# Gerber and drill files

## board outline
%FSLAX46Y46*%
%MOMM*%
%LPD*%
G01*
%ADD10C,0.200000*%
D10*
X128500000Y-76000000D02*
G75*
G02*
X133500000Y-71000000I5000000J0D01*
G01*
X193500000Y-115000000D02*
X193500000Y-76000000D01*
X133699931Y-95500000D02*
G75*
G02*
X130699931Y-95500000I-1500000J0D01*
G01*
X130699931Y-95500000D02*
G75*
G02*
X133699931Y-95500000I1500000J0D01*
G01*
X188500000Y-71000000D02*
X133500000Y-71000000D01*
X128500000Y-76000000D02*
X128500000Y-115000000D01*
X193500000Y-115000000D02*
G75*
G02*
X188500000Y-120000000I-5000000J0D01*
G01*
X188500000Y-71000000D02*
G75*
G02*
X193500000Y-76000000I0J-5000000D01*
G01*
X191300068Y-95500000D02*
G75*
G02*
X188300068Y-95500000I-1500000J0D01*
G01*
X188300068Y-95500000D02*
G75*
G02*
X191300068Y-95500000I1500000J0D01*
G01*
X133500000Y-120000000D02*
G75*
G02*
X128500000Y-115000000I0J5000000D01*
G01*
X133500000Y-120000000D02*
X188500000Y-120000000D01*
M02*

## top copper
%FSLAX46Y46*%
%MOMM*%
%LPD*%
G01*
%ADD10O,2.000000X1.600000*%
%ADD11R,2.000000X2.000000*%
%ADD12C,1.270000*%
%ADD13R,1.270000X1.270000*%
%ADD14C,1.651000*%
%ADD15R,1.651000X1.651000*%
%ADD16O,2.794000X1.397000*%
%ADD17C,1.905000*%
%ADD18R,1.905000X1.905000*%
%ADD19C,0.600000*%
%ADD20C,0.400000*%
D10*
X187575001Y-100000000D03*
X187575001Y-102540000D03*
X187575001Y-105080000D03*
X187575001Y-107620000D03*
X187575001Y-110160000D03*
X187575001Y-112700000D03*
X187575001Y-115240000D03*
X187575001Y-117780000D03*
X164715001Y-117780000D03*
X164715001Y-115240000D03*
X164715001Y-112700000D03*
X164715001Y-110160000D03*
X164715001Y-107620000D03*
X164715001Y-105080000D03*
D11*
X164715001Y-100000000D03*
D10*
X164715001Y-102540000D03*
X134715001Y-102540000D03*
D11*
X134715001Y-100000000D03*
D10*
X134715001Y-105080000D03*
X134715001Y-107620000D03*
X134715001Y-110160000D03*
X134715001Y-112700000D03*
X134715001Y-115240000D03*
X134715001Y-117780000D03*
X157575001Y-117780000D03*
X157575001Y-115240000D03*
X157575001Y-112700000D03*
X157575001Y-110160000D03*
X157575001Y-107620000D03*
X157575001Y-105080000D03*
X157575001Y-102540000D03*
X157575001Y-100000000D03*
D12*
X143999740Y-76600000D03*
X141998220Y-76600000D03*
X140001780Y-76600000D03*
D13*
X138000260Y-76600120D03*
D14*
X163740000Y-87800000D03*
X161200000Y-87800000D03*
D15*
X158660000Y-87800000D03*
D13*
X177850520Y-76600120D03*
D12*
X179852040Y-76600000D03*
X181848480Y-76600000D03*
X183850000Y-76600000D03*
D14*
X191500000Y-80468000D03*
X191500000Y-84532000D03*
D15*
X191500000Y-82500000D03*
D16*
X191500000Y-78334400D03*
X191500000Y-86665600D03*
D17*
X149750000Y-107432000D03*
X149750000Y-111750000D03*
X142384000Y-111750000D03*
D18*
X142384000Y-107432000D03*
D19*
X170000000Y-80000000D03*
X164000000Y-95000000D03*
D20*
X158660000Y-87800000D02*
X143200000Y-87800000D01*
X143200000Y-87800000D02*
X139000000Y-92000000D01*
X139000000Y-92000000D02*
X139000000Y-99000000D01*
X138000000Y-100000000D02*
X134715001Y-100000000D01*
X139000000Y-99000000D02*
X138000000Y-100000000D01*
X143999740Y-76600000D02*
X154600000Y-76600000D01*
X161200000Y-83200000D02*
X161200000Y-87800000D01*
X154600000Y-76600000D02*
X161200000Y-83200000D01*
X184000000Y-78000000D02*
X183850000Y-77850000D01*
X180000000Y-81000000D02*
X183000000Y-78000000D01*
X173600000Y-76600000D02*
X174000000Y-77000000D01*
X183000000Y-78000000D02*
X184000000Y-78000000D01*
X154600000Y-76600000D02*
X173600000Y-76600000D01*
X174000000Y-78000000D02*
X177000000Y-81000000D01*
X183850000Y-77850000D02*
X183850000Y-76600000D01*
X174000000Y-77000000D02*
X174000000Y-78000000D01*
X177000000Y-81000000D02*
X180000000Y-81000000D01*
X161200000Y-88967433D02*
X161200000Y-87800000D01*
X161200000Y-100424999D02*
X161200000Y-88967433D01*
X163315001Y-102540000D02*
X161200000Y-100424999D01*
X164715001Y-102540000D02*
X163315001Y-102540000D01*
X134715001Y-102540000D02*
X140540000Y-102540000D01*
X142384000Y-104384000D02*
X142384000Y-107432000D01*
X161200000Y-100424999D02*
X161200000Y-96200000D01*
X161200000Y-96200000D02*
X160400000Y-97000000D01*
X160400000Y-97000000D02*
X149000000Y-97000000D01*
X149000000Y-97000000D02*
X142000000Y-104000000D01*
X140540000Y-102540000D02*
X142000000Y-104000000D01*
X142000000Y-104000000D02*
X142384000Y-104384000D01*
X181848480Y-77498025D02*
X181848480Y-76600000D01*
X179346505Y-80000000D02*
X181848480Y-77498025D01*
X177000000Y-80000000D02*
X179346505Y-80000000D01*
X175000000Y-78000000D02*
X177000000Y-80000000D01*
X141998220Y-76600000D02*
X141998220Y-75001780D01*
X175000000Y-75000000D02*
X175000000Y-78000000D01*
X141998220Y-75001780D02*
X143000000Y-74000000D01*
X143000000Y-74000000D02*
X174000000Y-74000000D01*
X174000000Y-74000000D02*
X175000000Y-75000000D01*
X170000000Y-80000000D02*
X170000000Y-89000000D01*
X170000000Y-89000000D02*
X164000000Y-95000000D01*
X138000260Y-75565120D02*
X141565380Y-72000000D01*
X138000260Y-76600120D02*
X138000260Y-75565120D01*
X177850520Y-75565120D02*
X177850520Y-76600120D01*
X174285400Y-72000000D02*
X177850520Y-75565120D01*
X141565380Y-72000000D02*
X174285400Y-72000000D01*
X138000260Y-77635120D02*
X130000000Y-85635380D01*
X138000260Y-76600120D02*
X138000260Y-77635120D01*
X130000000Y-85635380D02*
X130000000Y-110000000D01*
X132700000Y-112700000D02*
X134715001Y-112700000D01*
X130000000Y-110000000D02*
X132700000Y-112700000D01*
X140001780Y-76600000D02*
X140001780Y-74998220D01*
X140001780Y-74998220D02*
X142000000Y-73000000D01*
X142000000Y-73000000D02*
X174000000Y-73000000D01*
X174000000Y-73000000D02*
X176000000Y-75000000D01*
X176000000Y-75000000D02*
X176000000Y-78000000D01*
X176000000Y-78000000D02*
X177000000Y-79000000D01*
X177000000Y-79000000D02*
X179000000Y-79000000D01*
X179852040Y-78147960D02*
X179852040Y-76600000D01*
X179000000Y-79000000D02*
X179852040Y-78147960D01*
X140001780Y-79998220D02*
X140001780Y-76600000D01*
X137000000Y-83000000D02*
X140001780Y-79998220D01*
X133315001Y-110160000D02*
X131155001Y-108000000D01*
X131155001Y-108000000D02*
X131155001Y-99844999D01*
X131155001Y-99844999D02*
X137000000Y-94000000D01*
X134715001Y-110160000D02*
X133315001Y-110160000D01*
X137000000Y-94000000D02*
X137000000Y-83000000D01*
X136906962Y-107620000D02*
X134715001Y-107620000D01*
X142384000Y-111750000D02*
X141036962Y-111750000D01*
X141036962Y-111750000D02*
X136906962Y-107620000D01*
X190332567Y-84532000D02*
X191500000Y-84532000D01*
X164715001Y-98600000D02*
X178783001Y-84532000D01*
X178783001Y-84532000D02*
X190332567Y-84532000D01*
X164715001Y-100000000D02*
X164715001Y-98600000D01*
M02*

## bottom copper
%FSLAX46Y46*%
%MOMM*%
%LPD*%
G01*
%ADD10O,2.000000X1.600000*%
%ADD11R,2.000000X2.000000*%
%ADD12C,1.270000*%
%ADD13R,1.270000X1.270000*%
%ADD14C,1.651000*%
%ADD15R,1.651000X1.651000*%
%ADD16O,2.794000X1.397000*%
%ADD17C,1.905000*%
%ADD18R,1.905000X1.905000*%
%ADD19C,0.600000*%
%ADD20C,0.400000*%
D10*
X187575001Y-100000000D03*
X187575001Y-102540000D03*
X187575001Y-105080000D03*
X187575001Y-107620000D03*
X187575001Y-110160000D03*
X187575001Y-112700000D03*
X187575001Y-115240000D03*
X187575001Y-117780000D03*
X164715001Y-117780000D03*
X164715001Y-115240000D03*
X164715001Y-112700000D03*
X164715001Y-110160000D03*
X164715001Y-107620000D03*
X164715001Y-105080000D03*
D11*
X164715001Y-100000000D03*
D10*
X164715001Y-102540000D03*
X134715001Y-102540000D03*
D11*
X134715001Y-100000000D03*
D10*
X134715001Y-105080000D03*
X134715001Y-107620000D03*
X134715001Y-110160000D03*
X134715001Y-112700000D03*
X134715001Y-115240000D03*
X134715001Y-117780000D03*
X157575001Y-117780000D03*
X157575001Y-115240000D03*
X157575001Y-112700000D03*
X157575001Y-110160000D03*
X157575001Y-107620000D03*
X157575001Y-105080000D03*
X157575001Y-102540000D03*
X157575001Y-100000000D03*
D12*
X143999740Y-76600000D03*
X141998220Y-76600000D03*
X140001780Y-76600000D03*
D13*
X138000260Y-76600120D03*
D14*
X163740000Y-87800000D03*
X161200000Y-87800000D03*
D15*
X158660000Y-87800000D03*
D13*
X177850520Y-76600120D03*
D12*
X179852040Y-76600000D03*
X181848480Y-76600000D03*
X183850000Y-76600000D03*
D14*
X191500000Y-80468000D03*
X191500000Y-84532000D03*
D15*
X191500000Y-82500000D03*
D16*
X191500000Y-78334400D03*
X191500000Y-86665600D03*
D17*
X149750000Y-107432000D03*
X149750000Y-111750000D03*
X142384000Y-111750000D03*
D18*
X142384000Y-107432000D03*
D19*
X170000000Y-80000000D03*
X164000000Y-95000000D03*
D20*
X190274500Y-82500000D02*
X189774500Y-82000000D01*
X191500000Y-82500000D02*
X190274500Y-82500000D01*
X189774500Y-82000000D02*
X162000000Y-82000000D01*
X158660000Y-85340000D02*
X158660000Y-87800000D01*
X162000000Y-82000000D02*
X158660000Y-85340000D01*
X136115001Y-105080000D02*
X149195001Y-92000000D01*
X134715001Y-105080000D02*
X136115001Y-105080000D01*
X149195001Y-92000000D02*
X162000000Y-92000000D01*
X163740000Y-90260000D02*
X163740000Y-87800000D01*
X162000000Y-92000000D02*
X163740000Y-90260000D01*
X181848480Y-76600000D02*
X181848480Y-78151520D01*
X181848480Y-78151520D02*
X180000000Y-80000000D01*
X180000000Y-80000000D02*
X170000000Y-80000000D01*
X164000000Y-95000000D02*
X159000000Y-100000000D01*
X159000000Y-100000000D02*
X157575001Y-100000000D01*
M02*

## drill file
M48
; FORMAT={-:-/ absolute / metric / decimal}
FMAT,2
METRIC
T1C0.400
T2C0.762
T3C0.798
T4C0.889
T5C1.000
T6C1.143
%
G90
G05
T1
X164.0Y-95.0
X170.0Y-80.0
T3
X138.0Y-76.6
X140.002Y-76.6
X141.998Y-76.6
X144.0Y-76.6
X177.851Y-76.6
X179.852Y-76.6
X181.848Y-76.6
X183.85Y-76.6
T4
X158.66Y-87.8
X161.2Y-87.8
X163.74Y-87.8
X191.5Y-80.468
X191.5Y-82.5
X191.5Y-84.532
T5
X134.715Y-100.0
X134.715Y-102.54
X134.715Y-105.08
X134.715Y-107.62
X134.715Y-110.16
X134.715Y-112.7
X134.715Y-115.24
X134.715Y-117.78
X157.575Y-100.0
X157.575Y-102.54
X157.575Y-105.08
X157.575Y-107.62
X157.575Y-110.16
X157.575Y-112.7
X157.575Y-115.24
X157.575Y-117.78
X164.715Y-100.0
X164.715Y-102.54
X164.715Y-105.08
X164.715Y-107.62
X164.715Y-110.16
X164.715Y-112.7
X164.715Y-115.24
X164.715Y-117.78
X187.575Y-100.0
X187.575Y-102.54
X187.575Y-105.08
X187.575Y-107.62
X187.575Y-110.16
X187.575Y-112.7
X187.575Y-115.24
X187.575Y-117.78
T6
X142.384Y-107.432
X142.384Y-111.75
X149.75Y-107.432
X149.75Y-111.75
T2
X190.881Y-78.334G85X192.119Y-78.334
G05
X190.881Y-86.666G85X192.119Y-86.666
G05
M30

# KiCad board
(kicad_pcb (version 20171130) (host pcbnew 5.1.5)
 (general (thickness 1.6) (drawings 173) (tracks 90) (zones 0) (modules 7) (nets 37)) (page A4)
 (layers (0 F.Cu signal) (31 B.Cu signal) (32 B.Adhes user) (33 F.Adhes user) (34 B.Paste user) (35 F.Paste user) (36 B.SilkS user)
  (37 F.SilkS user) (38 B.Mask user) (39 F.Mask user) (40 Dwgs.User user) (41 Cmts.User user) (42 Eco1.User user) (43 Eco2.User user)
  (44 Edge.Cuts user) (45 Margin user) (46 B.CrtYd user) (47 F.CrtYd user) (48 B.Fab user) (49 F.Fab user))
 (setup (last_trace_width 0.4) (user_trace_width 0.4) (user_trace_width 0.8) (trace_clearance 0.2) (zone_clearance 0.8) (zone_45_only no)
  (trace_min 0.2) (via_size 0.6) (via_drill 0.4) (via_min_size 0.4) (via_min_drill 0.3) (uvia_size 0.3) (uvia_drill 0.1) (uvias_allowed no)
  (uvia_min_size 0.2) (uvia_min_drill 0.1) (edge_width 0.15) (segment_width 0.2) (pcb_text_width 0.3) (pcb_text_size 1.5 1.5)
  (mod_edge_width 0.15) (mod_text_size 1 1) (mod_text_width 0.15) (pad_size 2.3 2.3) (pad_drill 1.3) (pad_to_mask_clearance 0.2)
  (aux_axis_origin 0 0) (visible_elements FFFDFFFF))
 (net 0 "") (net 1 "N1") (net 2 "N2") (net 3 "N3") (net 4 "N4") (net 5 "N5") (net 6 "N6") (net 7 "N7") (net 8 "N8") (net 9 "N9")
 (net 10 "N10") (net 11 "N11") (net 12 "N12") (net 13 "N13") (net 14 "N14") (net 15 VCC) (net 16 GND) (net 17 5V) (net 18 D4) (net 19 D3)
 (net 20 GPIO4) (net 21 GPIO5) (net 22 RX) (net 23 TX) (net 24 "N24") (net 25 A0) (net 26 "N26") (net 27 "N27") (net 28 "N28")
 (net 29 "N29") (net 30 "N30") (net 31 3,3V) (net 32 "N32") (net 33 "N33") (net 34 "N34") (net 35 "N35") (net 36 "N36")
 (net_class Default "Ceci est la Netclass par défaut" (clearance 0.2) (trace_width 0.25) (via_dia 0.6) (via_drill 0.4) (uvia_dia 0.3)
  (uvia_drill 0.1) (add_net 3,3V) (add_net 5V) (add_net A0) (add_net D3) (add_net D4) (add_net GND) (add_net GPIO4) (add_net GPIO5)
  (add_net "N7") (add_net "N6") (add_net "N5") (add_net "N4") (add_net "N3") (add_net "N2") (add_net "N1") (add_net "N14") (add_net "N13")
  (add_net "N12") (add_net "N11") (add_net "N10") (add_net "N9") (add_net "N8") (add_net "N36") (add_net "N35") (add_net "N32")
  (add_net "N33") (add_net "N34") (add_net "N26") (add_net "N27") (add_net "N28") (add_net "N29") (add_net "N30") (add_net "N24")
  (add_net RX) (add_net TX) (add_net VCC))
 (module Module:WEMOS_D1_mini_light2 (layer F.Cu) (at 164.715001 100)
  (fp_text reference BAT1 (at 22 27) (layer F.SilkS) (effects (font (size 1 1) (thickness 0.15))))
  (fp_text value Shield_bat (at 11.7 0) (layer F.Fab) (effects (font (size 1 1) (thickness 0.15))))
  (pad 16 thru_hole oval (at 22.86 0) (size 2 1.6) (drill 1) (layers *.Cu *.Mask) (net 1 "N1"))
  (pad 15 thru_hole oval (at 22.86 2.54) (size 2 1.6) (drill 1) (layers *.Cu *.Mask) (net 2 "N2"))
  (pad 14 thru_hole oval (at 22.86 5.08) (size 2 1.6) (drill 1) (layers *.Cu *.Mask) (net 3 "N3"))
  (pad 13 thru_hole oval (at 22.86 7.62) (size 2 1.6) (drill 1) (layers *.Cu *.Mask) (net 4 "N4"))
  (pad 12 thru_hole oval (at 22.86 10.16) (size 2 1.6) (drill 1) (layers *.Cu *.Mask) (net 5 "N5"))
  (pad 11 thru_hole oval (at 22.86 12.7) (size 2 1.6) (drill 1) (layers *.Cu *.Mask) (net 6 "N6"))
  (pad 10 thru_hole oval (at 22.86 15.24) (size 2 1.6) (drill 1) (layers *.Cu *.Mask) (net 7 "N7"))
  (pad 9 thru_hole oval (at 22.86 17.78) (size 2 1.6) (drill 1) (layers *.Cu *.Mask) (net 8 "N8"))
  (pad 8 thru_hole oval (at 0 17.78) (size 2 1.6) (drill 1) (layers *.Cu *.Mask) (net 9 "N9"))
  (pad 7 thru_hole oval (at 0 15.24) (size 2 1.6) (drill 1) (layers *.Cu *.Mask) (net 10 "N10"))
  (pad 6 thru_hole oval (at 0 12.7) (size 2 1.6) (drill 1) (layers *.Cu *.Mask) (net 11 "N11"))
  (pad 5 thru_hole oval (at 0 10.16) (size 2 1.6) (drill 1) (layers *.Cu *.Mask) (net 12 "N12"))
  (pad 4 thru_hole oval (at 0 7.62) (size 2 1.6) (drill 1) (layers *.Cu *.Mask) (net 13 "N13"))
  (pad 3 thru_hole oval (at 0 5.08) (size 2 1.6) (drill 1) (layers *.Cu *.Mask) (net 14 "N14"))
  (pad 1 thru_hole rect (at 0 0) (size 2 2) (drill 1) (layers *.Cu *.Mask) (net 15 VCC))
  (pad 2 thru_hole oval (at 0 2.54) (size 2 1.6) (drill 1) (layers *.Cu *.Mask) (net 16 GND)))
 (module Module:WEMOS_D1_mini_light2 (layer F.Cu) (at 134.715001 100)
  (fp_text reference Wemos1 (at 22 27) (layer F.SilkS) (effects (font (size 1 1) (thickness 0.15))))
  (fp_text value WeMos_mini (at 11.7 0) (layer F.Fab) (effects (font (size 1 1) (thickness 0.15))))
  (pad 2 thru_hole oval (at 0 2.54) (size 2 1.6) (drill 1) (layers *.Cu *.Mask) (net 16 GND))
  (pad 1 thru_hole rect (at 0 0) (size 2 2) (drill 1) (layers *.Cu *.Mask) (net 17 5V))
  (pad 3 thru_hole oval (at 0 5.08) (size 2 1.6) (drill 1) (layers *.Cu *.Mask) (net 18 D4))
  (pad 4 thru_hole oval (at 0 7.62) (size 2 1.6) (drill 1) (layers *.Cu *.Mask) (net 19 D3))
  (pad 5 thru_hole oval (at 0 10.16) (size 2 1.6) (drill 1) (layers *.Cu *.Mask) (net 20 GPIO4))
  (pad 6 thru_hole oval (at 0 12.7) (size 2 1.6) (drill 1) (layers *.Cu *.Mask) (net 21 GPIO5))
  (pad 7 thru_hole oval (at 0 15.24) (size 2 1.6) (drill 1) (layers *.Cu *.Mask) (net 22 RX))
  (pad 8 thru_hole oval (at 0 17.78) (size 2 1.6) (drill 1) (layers *.Cu *.Mask) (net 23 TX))
  (pad 9 thru_hole oval (at 22.86 17.78) (size 2 1.6) (drill 1) (layers *.Cu *.Mask) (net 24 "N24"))
  (pad 10 thru_hole oval (at 22.86 15.24) (size 2 1.6) (drill 1) (layers *.Cu *.Mask) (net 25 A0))
  (pad 11 thru_hole oval (at 22.86 12.7) (size 2 1.6) (drill 1) (layers *.Cu *.Mask) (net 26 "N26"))
  (pad 12 thru_hole oval (at 22.86 10.16) (size 2 1.6) (drill 1) (layers *.Cu *.Mask) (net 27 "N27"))
  (pad 13 thru_hole oval (at 22.86 7.62) (size 2 1.6) (drill 1) (layers *.Cu *.Mask) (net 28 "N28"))
  (pad 14 thru_hole oval (at 22.86 5.08) (size 2 1.6) (drill 1) (layers *.Cu *.Mask) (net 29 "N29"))
  (pad 15 thru_hole oval (at 22.86 2.54) (size 2 1.6) (drill 1) (layers *.Cu *.Mask) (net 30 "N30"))
  (pad 16 thru_hole oval (at 22.86 0) (size 2 1.6) (drill 1) (layers *.Cu *.Mask) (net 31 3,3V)))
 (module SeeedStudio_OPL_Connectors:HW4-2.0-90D (layer F.Cu) (at 141 73.4)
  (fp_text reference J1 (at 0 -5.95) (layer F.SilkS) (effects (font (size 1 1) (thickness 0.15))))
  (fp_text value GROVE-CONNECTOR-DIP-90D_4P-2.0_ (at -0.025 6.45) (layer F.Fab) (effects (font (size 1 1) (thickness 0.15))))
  (pad 4 thru_hole circle (at 2.99974 3.2) (size 1.27 1.27) (drill 0.79756) (layers *.Cu *.Mask) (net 16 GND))
  (pad 3 thru_hole circle (at 0.99822 3.2) (size 1.27 1.27) (drill 0.79756) (layers *.Cu *.Mask) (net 31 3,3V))
  (pad 2 thru_hole circle (at -0.99822 3.2) (size 1.27 1.27) (drill 0.79756) (layers *.Cu *.Mask) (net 20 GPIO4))
  (pad 1 thru_hole rect (at -2.99974 3.20012) (size 1.27 1.27) (drill 0.79756) (layers *.Cu *.Mask) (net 21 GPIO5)))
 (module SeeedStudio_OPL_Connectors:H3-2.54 (layer F.Cu) (at 161.2 87.8 180)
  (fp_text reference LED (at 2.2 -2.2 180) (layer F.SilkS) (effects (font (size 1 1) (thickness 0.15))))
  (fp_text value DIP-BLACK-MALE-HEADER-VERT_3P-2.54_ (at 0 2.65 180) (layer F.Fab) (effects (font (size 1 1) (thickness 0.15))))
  (pad 3 thru_hole circle (at -2.54 0 270) (size 1.651 1.651) (drill 0.889) (layers *.Cu *.Mask) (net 18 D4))
  (pad 2 thru_hole circle (at 0 0 270) (size 1.651 1.651) (drill 0.889) (layers *.Cu *.Mask) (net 16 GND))
  (pad 1 thru_hole rect (at 2.54 0 270) (size 1.651 1.651) (drill 0.889) (layers *.Cu *.Mask) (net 17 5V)))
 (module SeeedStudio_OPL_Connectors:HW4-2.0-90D (layer F.Cu) (at 180.85026 73.4)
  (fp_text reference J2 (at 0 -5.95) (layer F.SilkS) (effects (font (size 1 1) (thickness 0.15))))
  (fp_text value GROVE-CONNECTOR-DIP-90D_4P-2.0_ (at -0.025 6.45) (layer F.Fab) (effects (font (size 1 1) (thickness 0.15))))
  (pad 1 thru_hole rect (at -2.99974 3.20012) (size 1.27 1.27) (drill 0.79756) (layers *.Cu *.Mask) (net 21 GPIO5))
  (pad 2 thru_hole circle (at -0.99822 3.2) (size 1.27 1.27) (drill 0.79756) (layers *.Cu *.Mask) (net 20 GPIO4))
  (pad 3 thru_hole circle (at 0.99822 3.2) (size 1.27 1.27) (drill 0.79756) (layers *.Cu *.Mask) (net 31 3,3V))
  (pad 4 thru_hole circle (at 2.99974 3.2) (size 1.27 1.27) (drill 0.79756) (layers *.Cu *.Mask) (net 16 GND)))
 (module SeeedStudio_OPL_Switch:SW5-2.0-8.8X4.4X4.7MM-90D (layer F.Cu) (at 191.5 82.5)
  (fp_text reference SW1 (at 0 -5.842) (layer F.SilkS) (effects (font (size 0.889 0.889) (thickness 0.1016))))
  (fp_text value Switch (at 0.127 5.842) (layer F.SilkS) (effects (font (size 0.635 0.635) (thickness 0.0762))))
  (pad A thru_hole circle (at 0 -2.032) (size 1.651 1.651) (drill 0.889) (layers *.Cu *.Mask) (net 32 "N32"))
  (pad B thru_hole circle (at 0 2.032) (size 1.651 1.651) (drill 0.889) (layers *.Cu *.Mask) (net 15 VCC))
  (pad COM thru_hole rect (at 0 0) (size 1.651 1.651) (drill 0.889) (layers *.Cu *.Mask) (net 17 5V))
  (pad NC1 thru_hole oval (at 0 -4.1656 90) (size 1.397 2.794) (drill oval 0.762 2) (layers *.Cu *.Mask) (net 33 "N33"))
  (pad NC2 thru_hole oval (at 0 4.1656 90) (size 1.397 2.794) (drill oval 0.762 2) (layers *.Cu *.Mask) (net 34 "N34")))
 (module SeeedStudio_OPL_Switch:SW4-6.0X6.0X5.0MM (layer F.Cu) (at 146.067 109.591)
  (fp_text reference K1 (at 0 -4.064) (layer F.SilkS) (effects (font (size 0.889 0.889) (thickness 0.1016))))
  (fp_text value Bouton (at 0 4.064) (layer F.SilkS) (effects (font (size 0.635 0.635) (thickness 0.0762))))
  (pad 4 thru_hole circle (at 3.683 -2.159) (size 1.905 1.905) (drill 1.143) (layers *.Cu *.Mask) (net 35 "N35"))
  (pad 3 thru_hole circle (at 3.683 2.159) (size 1.905 1.905) (drill 1.143) (layers *.Cu *.Mask) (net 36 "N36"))
  (pad 2 thru_hole circle (at -3.683 2.159) (size 1.905 1.905) (drill 1.143) (layers *.Cu *.Mask) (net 19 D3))
  (pad 1 thru_hole rect (at -3.683 -2.159) (size 1.905 1.905) (drill 1.143) (layers *.Cu *.Mask) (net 16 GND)))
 (gr_arc (start 133.5 76) (end 133.5 71) (angle -90) (layer Edge.Cuts) (width 0.2))
 (gr_line (start 193.5 115) (end 193.5 76) (layer Edge.Cuts) (width 0.2))
 (gr_circle (center 132.199931 95.5) (end 133.699931 95.5) (layer Edge.Cuts) (width 0.2))
 (gr_line (start 188.5 71) (end 133.5 71) (layer Edge.Cuts) (width 0.2))
 (gr_line (start 128.5 76) (end 128.5 115) (layer Edge.Cuts) (width 0.2))
 (gr_arc (start 188.5 115) (end 188.5 120) (angle -90) (layer Edge.Cuts) (width 0.2))
 (gr_arc (start 188.5 76) (end 193.5 76) (angle -90) (layer Edge.Cuts) (width 0.2))
 (gr_circle (center 189.800068 95.5) (end 191.300068 95.5) (layer Edge.Cuts) (width 0.2))
 (gr_arc (start 133.5 115) (end 128.5 115) (angle -90) (layer Edge.Cuts) (width 0.2))
 (gr_line (start 133.5 120) (end 188.5 120) (layer Edge.Cuts) (width 0.2))
 (segment (start 158.66 87.8) (end 143.2 87.8) (width 0.4) (layer F.Cu) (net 17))
 (segment (start 143.2 87.8) (end 139 92) (width 0.4) (layer F.Cu) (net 17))
 (segment (start 139 92) (end 139 99) (width 0.4) (layer F.Cu) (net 17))
 (segment (start 138 100) (end 134.715001 100) (width 0.4) (layer F.Cu) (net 17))
 (segment (start 139 99) (end 138 100) (width 0.4) (layer F.Cu) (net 17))
 (segment (start 190.2745 82.5) (end 189.7745 82) (width 0.4) (layer B.Cu) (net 17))
 (segment (start 191.5 82.5) (end 190.2745 82.5) (width 0.4) (layer B.Cu) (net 17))
 (segment (start 189.7745 82) (end 162 82) (width 0.4) (layer B.Cu) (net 17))
 (segment (start 158.66 85.34) (end 158.66 87.8) (width 0.4) (layer B.Cu) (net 17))
 (segment (start 162 82) (end 158.66 85.34) (width 0.4) (layer B.Cu) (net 17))
 (segment (start 136.115001 105.08) (end 149.195001 92) (width 0.4) (layer B.Cu) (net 18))
 (segment (start 134.715001 105.08) (end 136.115001 105.08) (width 0.4) (layer B.Cu) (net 18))
 (segment (start 149.195001 92) (end 162 92) (width 0.4) (layer B.Cu) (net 18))
 (segment (start 163.74 90.26) (end 163.74 87.8) (width 0.4) (layer B.Cu) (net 18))
 (segment (start 162 92) (end 163.74 90.26) (width 0.4) (layer B.Cu) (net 18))
 (segment (start 143.99974 76.6) (end 154.6 76.6) (width 0.4) (layer F.Cu) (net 16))
 (segment (start 161.2 83.2) (end 161.2 87.8) (width 0.4) (layer F.Cu) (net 16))
 (segment (start 154.6 76.6) (end 161.2 83.2) (width 0.4) (layer F.Cu) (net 16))
 (segment (start 184 78) (end 183.85 77.85) (width 0.4) (layer F.Cu) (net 16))
 (segment (start 180 81) (end 183 78) (width 0.4) (layer F.Cu) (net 16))
 (segment (start 173.6 76.6) (end 174 77) (width 0.4) (layer F.Cu) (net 16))
 (segment (start 183 78) (end 184 78) (width 0.4) (layer F.Cu) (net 16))
 (segment (start 154.6 76.6) (end 173.6 76.6) (width 0.4) (layer F.Cu) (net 16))
 (segment (start 174 78) (end 177 81) (width 0.4) (layer F.Cu) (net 16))
 (segment (start 183.85 77.85) (end 183.85 76.6) (width 0.4) (layer F.Cu) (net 16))
 (segment (start 174 77) (end 174 78) (width 0.4) (layer F.Cu) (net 16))
 (segment (start 177 81) (end 180 81) (width 0.4) (layer F.Cu) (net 16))
 (segment (start 161.2 88.967433) (end 161.2 87.8) (width 0.4) (layer F.Cu) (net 16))
 (segment (start 161.2 100.424999) (end 161.2 88.967433) (width 0.4) (layer F.Cu) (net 16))
 (segment (start 163.315001 102.54) (end 161.2 100.424999) (width 0.4) (layer F.Cu) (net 16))
 (segment (start 164.715001 102.54) (end 163.315001 102.54) (width 0.4) (layer F.Cu) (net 16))
 (segment (start 134.715001 102.54) (end 140.54 102.54) (width 0.4) (layer F.Cu) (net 16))
 (segment (start 142.384 104.384) (end 142.384 107.432) (width 0.4) (layer F.Cu) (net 16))
 (segment (start 161.2 100.424999) (end 161.2 96.2) (width 0.4) (layer F.Cu) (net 16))
 (segment (start 161.2 96.2) (end 160.4 97) (width 0.4) (layer F.Cu) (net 16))
 (segment (start 160.4 97) (end 149 97) (width 0.4) (layer F.Cu) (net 16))
 (segment (start 149 97) (end 142 104) (width 0.4) (layer F.Cu) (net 16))
 (segment (start 140.54 102.54) (end 142 104) (width 0.4) (layer F.Cu) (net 16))
 (segment (start 142 104) (end 142.384 104.384) (width 0.4) (layer F.Cu) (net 16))
 (segment (start 181.84848 77.498025) (end 181.84848 76.6) (width 0.4) (layer F.Cu) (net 31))
 (segment (start 179.346505 80) (end 181.84848 77.498025) (width 0.4) (layer F.Cu) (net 31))
 (segment (start 177 80) (end 179.346505 80) (width 0.4) (layer F.Cu) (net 31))
 (segment (start 175 78) (end 177 80) (width 0.4) (layer F.Cu) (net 31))
 (segment (start 141.99822 76.6) (end 141.99822 75.00178) (width 0.4) (layer F.Cu) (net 31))
 (segment (start 175 75) (end 175 78) (width 0.4) (layer F.Cu) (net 31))
 (segment (start 141.99822 75.00178) (end 143 74) (width 0.4) (layer F.Cu) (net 31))
 (segment (start 143 74) (end 174 74) (width 0.4) (layer F.Cu) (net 31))
 (segment (start 174 74) (end 175 75) (width 0.4) (layer F.Cu) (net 31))
 (segment (start 181.84848 76.6) (end 181.84848 78.15152) (width 0.4) (layer B.Cu) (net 31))
 (segment (start 181.84848 78.15152) (end 180 80) (width 0.4) (layer B.Cu) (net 31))
 (segment (start 180 80) (end 170 80) (width 0.4) (layer B.Cu) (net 31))
 (via (at 170 80) (size 0.6) (drill 0.4) (layers F.Cu B.Cu) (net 31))
 (segment (start 170 80) (end 170 89) (width 0.4) (layer F.Cu) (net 31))
 (via (at 164 95) (size 0.6) (drill 0.4) (layers F.Cu B.Cu) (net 31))
 (segment (start 170 89) (end 164 95) (width 0.4) (layer F.Cu) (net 31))
 (segment (start 164 95) (end 159 100) (width 0.4) (layer B.Cu) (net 31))
 (segment (start 159 100) (end 157.575001 100) (width 0.4) (layer B.Cu) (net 31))
 (segment (start 138.00026 75.56512) (end 141.56538 72) (width 0.4) (layer F.Cu) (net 21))
 (segment (start 138.00026 76.60012) (end 138.00026 75.56512) (width 0.4) (layer F.Cu) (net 21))
 (segment (start 177.85052 75.56512) (end 177.85052 76.60012) (width 0.4) (layer F.Cu) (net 21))
 (segment (start 174.2854 72) (end 177.85052 75.56512) (width 0.4) (layer F.Cu) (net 21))
 (segment (start 141.56538 72) (end 174.2854 72) (width 0.4) (layer F.Cu) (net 21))
 (segment (start 138.00026 77.63512) (end 130 85.63538) (width 0.4) (layer F.Cu) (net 21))
 (segment (start 138.00026 76.60012) (end 138.00026 77.63512) (width 0.4) (layer F.Cu) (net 21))
 (segment (start 130 85.63538) (end 130 110) (width 0.4) (layer F.Cu) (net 21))
 (segment (start 132.7 112.7) (end 134.715001 112.7) (width 0.4) (layer F.Cu) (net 21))
 (segment (start 130 110) (end 132.7 112.7) (width 0.4) (layer F.Cu) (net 21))
 (segment (start 140.00178 76.6) (end 140.00178 74.99822) (width 0.4) (layer F.Cu) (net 20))
 (segment (start 140.00178 74.99822) (end 142 73) (width 0.4) (layer F.Cu) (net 20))
 (segment (start 142 73) (end 174 73) (width 0.4) (layer F.Cu) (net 20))
 (segment (start 174 73) (end 176 75) (width 0.4) (layer F.Cu) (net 20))
 (segment (start 176 75) (end 176 78) (width 0.4) (layer F.Cu) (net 20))
 (segment (start 176 78) (end 177 79) (width 0.4) (layer F.Cu) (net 20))
 (segment (start 177 79) (end 179 79) (width 0.4) (layer F.Cu) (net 20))
 (segment (start 179.85204 78.14796) (end 179.85204 76.6) (width 0.4) (layer F.Cu) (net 20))
 (segment (start 179 79) (end 179.85204 78.14796) (width 0.4) (layer F.Cu) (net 20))
 (segment (start 140.00178 79.99822) (end 140.00178 76.6) (width 0.4) (layer F.Cu) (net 20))
 (segment (start 137 83) (end 140.00178 79.99822) (width 0.4) (layer F.Cu) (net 20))
 (segment (start 133.315001 110.16) (end 131.155001 108) (width 0.4) (layer F.Cu) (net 20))
 (segment (start 131.155001 108) (end 131.155001 99.844999) (width 0.4) (layer F.Cu) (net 20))
 (segment (start 131.155001 99.844999) (end 137 94) (width 0.4) (layer F.Cu) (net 20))
 (segment (start 134.715001 110.16) (end 133.315001 110.16) (width 0.4) (layer F.Cu) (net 20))
 (segment (start 137 94) (end 137 83) (width 0.4) (layer F.Cu) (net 20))
 (segment (start 136.906962 107.62) (end 134.715001 107.62) (width 0.4) (layer F.Cu) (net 19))
 (segment (start 142.384 111.75) (end 141.036962 111.75) (width 0.4) (layer F.Cu) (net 19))
 (segment (start 141.036962 111.75) (end 136.906962 107.62) (width 0.4) (layer F.Cu) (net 19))
 (segment (start 190.332567 84.532) (end 191.5 84.532) (width 0.4) (layer F.Cu) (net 15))
 (segment (start 164.715001 98.6) (end 178.783001 84.532) (width 0.4) (layer F.Cu) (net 15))
 (segment (start 178.783001 84.532) (end 190.332567 84.532) (width 0.4) (layer F.Cu) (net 15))
 (segment (start 164.715001 100) (end 164.715001 98.6) (width 0.4) (layer F.Cu) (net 15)))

